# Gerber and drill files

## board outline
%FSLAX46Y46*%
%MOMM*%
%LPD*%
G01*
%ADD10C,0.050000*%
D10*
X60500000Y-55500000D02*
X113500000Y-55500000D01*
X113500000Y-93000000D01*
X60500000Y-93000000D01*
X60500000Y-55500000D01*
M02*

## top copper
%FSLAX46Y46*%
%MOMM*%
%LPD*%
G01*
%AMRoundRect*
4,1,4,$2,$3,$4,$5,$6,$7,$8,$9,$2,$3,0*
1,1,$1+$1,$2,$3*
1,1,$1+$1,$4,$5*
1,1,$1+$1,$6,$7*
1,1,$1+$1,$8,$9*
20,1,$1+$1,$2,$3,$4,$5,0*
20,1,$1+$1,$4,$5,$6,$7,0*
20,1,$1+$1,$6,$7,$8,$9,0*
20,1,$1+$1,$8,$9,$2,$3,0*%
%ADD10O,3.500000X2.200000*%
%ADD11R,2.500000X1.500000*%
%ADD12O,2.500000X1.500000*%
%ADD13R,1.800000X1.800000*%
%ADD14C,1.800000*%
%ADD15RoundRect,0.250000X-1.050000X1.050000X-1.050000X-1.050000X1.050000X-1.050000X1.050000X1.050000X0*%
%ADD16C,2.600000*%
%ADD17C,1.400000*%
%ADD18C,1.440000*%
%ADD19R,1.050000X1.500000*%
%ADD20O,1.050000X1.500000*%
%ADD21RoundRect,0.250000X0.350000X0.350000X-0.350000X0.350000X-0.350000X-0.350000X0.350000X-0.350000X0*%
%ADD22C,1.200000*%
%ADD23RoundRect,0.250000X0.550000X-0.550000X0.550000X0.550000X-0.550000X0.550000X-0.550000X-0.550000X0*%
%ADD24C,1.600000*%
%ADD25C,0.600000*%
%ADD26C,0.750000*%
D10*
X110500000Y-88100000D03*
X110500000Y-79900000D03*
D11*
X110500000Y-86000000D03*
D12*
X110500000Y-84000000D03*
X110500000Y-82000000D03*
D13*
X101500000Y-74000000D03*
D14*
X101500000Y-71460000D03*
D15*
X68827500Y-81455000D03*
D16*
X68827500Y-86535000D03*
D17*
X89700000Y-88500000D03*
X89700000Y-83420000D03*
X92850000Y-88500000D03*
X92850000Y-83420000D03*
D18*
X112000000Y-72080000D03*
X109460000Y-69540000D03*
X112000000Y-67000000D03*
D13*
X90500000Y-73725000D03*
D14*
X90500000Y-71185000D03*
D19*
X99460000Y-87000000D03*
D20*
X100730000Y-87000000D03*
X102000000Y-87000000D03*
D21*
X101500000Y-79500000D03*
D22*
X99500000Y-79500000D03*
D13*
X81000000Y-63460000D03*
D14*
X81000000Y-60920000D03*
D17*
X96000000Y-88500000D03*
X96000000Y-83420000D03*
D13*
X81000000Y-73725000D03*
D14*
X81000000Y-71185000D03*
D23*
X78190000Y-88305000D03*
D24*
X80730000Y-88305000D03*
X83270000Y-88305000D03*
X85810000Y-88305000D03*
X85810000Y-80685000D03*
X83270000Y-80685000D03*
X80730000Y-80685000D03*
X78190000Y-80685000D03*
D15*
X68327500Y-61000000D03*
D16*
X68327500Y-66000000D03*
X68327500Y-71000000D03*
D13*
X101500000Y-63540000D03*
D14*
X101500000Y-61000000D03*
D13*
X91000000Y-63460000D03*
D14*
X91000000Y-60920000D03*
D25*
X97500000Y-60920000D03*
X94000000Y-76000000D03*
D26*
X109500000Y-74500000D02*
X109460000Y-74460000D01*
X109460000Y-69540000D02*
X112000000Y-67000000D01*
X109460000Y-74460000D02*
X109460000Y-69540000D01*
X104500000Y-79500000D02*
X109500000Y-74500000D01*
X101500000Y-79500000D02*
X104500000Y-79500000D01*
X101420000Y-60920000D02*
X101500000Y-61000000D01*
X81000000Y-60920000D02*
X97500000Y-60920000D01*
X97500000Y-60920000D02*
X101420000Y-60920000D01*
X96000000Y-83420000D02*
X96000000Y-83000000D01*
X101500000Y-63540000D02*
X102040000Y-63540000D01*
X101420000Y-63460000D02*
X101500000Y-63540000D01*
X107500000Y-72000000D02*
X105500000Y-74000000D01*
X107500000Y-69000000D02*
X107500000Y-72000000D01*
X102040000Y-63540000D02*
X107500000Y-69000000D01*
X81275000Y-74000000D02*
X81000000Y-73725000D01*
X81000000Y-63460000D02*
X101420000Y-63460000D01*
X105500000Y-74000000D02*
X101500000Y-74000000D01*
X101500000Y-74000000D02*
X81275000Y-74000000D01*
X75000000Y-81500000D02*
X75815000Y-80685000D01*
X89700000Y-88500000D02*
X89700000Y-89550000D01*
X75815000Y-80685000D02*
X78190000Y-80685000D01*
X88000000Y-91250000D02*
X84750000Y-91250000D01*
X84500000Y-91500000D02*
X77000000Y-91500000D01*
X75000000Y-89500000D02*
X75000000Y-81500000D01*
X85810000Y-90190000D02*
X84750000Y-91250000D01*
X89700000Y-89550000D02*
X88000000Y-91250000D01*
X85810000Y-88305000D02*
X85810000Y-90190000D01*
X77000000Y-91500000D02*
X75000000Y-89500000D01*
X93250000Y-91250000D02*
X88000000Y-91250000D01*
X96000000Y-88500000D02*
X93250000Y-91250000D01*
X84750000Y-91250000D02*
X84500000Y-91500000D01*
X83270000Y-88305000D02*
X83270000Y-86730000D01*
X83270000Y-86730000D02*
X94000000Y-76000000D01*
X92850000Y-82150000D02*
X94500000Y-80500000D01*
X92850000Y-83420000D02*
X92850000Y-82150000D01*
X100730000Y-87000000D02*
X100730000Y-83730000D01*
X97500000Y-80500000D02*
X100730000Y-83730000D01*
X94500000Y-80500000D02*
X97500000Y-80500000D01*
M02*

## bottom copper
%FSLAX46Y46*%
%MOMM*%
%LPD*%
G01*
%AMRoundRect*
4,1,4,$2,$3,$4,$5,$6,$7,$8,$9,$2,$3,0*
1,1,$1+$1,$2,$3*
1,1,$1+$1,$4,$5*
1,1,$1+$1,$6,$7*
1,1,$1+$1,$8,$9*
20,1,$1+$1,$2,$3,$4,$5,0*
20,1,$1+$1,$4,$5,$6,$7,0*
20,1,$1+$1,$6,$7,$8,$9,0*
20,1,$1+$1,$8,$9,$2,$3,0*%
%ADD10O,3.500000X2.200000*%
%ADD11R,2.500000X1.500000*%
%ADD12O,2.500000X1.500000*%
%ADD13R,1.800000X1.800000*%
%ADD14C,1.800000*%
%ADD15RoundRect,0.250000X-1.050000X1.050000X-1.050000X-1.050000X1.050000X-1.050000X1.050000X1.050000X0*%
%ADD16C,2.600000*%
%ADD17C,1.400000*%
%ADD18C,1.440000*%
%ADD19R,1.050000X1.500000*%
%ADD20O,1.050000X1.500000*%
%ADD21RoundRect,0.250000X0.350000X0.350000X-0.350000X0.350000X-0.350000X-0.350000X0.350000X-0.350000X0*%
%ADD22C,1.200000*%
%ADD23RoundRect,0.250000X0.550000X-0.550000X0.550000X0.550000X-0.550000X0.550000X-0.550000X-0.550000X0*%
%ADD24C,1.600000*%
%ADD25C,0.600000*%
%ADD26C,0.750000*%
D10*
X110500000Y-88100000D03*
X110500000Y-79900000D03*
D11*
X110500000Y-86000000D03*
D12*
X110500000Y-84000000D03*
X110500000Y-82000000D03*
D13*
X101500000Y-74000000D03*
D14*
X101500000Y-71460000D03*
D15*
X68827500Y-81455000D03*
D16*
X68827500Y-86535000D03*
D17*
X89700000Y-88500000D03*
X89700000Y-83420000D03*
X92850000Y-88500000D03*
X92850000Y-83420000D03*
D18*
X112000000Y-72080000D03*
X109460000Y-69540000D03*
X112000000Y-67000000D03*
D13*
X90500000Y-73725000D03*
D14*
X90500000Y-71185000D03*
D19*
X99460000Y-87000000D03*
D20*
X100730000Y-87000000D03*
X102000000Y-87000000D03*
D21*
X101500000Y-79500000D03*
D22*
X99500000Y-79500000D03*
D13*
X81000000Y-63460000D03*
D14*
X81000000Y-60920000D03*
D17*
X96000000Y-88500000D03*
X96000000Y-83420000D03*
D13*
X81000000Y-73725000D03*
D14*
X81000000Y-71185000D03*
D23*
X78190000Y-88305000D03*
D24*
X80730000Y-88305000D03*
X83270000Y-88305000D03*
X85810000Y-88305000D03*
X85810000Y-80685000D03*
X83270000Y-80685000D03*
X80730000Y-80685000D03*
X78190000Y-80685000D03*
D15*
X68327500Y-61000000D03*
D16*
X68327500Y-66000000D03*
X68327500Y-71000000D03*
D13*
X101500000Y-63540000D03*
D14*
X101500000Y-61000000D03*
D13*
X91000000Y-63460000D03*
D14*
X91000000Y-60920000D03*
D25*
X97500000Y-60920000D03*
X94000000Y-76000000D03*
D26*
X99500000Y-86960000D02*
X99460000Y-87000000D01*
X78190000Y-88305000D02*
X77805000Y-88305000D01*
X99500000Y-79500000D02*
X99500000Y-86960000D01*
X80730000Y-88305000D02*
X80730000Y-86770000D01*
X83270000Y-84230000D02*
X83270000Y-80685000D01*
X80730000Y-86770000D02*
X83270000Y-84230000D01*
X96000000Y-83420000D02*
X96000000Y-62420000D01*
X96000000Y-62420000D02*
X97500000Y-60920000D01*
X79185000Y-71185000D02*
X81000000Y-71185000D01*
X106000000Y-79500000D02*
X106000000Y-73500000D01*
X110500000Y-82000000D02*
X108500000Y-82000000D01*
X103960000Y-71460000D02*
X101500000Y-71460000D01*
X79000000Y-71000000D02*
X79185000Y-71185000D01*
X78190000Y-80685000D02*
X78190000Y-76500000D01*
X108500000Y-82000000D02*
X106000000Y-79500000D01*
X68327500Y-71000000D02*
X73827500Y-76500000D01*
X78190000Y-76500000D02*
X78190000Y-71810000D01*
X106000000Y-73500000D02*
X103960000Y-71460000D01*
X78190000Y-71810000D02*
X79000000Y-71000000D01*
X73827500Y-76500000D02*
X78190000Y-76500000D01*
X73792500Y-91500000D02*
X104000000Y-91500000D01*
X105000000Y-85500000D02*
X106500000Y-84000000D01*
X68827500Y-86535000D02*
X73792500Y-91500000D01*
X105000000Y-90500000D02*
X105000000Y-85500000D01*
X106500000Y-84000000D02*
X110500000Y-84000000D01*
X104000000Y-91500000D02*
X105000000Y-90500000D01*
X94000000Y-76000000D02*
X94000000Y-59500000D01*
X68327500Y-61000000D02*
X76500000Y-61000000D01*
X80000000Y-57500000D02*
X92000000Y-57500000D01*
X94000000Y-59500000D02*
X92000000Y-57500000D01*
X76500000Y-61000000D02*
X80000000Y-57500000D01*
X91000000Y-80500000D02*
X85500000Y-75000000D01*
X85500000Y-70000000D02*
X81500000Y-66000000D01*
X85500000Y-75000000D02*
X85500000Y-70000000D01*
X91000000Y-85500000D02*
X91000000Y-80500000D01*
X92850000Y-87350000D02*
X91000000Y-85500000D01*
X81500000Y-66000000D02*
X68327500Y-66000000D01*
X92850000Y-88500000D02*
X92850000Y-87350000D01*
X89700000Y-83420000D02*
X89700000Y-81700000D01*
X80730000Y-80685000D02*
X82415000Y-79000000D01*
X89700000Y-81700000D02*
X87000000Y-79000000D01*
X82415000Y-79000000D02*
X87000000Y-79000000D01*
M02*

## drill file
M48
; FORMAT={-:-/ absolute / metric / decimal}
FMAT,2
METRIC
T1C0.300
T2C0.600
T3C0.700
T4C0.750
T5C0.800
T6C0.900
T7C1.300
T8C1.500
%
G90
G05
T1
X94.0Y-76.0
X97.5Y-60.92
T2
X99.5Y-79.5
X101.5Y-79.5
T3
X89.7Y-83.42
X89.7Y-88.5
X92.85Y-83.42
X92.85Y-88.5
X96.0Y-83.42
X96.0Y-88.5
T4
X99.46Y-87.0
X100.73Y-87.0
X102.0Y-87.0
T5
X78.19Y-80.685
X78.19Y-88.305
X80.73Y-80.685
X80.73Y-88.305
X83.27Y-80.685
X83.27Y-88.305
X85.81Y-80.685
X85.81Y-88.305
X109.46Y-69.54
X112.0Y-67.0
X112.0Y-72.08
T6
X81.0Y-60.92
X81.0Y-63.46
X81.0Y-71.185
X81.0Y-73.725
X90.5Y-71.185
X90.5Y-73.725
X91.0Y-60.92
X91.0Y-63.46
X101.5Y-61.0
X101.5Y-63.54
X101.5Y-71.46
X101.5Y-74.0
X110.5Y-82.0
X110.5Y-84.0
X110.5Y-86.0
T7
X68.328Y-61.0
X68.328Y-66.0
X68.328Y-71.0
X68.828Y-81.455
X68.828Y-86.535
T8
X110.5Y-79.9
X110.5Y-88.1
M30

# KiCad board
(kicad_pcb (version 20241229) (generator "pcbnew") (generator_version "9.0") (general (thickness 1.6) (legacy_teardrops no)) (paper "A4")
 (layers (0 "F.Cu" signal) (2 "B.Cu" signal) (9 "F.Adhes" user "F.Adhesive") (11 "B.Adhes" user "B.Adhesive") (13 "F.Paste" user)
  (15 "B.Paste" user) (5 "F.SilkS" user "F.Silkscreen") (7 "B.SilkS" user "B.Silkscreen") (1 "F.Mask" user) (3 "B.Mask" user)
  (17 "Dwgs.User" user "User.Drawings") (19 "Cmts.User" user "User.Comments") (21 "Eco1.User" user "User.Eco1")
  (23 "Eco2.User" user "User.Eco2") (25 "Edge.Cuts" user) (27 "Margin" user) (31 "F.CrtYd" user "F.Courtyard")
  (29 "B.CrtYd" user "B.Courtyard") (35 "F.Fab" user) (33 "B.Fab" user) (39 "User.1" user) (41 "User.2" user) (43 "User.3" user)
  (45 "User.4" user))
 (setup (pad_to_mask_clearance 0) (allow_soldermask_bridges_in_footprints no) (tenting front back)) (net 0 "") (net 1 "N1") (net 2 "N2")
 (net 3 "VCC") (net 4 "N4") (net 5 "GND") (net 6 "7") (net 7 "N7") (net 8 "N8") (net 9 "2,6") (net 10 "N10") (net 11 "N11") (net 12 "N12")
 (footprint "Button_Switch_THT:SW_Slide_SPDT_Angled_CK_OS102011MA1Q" (layer "F.Cu") (at 110.5 86 90)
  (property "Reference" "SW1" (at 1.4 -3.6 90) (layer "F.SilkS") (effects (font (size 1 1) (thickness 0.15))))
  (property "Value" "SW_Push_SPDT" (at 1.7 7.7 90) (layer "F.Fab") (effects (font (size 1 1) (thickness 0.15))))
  (pad "" thru_hole oval (at -2.1 0 90) (size 2.2 3.5) (drill 1.5) (layers "*.Cu" "*.Mask") (remove_unused_layers no))
  (pad "" thru_hole oval (at 6.1 0 90) (size 2.2 3.5) (drill 1.5) (layers "*.Cu" "*.Mask") (remove_unused_layers no))
  (pad "1" thru_hole rect (at 0 0 90) (size 1.5 2.5) (drill 0.9) (layers "*.Cu" "*.Mask") (remove_unused_layers no) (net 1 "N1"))
  (pad "2" thru_hole oval (at 2 0 90) (size 1.5 2.5) (drill 0.9) (layers "*.Cu" "*.Mask") (remove_unused_layers no) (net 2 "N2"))
  (pad "3" thru_hole oval (at 4 0 90) (size 1.5 2.5) (drill 0.9) (layers "*.Cu" "*.Mask") (remove_unused_layers no) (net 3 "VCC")))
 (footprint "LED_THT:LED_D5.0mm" (layer "F.Cu") (at 101.5 74 90)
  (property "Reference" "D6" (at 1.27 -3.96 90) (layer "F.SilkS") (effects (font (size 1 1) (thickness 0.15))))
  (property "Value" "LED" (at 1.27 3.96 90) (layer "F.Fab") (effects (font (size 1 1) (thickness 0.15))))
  (pad "1" thru_hole rect (at 0 0 90) (size 1.8 1.8) (drill 0.9) (layers "*.Cu" "*.Mask") (remove_unused_layers no) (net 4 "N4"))
  (pad "2" thru_hole circle (at 2.54 0 90) (size 1.8 1.8) (drill 0.9) (layers "*.Cu" "*.Mask") (remove_unused_layers no) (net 3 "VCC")))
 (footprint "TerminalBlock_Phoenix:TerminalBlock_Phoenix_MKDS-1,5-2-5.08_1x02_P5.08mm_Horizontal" (layer "F.Cu") (at 68.8275 81.455 -90)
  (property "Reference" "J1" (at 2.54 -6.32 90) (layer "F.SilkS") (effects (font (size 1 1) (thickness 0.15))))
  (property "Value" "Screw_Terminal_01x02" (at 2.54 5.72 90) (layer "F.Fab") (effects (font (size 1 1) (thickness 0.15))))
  (pad "1" thru_hole roundrect (at 0 0 270) (size 2.6 2.6) (drill 1.3) (layers "*.Cu" "*.Mask") (remove_unused_layers no)
   (roundrect_rratio 0.096154) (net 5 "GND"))
  (pad "2" thru_hole circle (at 5.08 0 270) (size 2.6 2.6) (drill 1.3) (layers "*.Cu" "*.Mask") (remove_unused_layers no) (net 2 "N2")))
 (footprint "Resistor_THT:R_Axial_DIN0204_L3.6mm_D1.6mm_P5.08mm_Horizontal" (layer "F.Cu") (at 89.7 88.5 90)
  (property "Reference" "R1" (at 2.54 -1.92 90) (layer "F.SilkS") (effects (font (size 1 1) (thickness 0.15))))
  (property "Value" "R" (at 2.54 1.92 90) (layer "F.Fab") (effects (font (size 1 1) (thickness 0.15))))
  (pad "1" thru_hole circle (at 0 0 90) (size 1.4 1.4) (drill 0.7) (layers "*.Cu" "*.Mask") (remove_unused_layers no) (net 3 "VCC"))
  (pad "2" thru_hole circle (at 5.08 0 90) (size 1.4 1.4) (drill 0.7) (layers "*.Cu" "*.Mask") (remove_unused_layers no) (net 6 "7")))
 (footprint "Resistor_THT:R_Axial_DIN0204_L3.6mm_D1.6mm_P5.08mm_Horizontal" (layer "F.Cu") (at 92.85 88.5 90)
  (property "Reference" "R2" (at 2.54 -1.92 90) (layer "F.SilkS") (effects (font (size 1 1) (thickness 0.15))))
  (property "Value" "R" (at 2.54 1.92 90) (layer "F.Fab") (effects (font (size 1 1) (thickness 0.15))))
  (pad "1" thru_hole circle (at 0 0 90) (size 1.4 1.4) (drill 0.7) (layers "*.Cu" "*.Mask") (remove_unused_layers no) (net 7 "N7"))
  (pad "2" thru_hole circle (at 5.08 0 90) (size 1.4 1.4) (drill 0.7) (layers "*.Cu" "*.Mask") (remove_unused_layers no) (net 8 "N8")))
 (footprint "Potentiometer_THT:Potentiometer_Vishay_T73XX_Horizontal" (layer "F.Cu") (at 112 72.08 180)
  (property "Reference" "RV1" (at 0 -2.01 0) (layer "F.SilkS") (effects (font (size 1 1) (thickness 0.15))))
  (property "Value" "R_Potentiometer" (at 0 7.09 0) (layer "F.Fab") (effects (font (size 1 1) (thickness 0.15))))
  (pad "1" thru_hole circle (at 0 0 180) (size 1.44 1.44) (drill 0.8) (layers "*.Cu" "*.Mask") (remove_unused_layers no) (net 6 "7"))
  (pad "2" thru_hole circle (at 2.54 2.54 180) (size 1.44 1.44) (drill 0.8) (layers "*.Cu" "*.Mask") (remove_unused_layers no) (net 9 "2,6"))
  (pad "3" thru_hole circle (at 0 5.08 180) (size 1.44 1.44) (drill 0.8) (layers "*.Cu" "*.Mask") (remove_unused_layers no) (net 9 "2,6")))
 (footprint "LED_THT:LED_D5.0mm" (layer "F.Cu") (at 90.5 73.725 90)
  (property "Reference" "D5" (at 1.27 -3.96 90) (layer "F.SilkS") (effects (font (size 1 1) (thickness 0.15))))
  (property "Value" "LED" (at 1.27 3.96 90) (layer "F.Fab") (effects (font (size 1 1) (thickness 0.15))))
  (pad "1" thru_hole rect (at 0 0 90) (size 1.8 1.8) (drill 0.9) (layers "*.Cu" "*.Mask") (remove_unused_layers no) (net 4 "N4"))
  (pad "2" thru_hole circle (at 2.54 0 90) (size 1.8 1.8) (drill 0.9) (layers "*.Cu" "*.Mask") (remove_unused_layers no) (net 3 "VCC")))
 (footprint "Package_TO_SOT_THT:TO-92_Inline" (layer "F.Cu") (at 99.46 87)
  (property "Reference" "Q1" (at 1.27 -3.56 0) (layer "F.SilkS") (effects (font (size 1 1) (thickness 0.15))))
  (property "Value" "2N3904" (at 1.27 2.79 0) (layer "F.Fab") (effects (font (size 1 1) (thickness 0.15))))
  (pad "1" thru_hole rect (at 0 0) (size 1.05 1.5) (drill 0.75) (layers "*.Cu" "*.Mask") (remove_unused_layers no) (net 5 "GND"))
  (pad "2" thru_hole oval (at 1.27 0) (size 1.05 1.5) (drill 0.75) (layers "*.Cu" "*.Mask") (remove_unused_layers no) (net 8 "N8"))
  (pad "3" thru_hole oval (at 2.54 0) (size 1.05 1.5) (drill 0.75) (layers "*.Cu" "*.Mask") (remove_unused_layers no) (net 4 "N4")))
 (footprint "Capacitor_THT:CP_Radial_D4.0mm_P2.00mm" (layer "F.Cu") (at 101.5 79.5 180)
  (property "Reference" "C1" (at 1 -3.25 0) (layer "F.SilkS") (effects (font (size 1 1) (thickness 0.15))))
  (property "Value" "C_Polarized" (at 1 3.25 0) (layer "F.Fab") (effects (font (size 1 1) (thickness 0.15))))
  (pad "1" thru_hole roundrect (at 0 0 180) (size 1.2 1.2) (drill 0.6) (layers "*.Cu" "*.Mask") (remove_unused_layers no)
   (roundrect_rratio 0.208333) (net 9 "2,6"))
  (pad "2" thru_hole circle (at 2 0 180) (size 1.2 1.2) (drill 0.6) (layers "*.Cu" "*.Mask") (remove_unused_layers no) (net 5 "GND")))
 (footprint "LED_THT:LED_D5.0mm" (layer "F.Cu") (at 81 63.46 90)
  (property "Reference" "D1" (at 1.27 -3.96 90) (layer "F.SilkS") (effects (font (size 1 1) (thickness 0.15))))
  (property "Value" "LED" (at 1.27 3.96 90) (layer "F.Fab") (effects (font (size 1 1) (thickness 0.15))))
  (pad "1" thru_hole rect (at 0 0 90) (size 1.8 1.8) (drill 0.9) (layers "*.Cu" "*.Mask") (remove_unused_layers no) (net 4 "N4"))
  (pad "2" thru_hole circle (at 2.54 0 90) (size 1.8 1.8) (drill 0.9) (layers "*.Cu" "*.Mask") (remove_unused_layers no) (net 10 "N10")))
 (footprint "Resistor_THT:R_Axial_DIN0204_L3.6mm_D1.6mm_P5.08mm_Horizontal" (layer "F.Cu") (at 96 88.5 90)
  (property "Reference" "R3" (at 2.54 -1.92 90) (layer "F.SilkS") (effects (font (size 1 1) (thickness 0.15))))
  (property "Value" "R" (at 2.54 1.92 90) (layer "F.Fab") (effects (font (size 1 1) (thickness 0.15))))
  (pad "1" thru_hole circle (at 0 0 90) (size 1.4 1.4) (drill 0.7) (layers "*.Cu" "*.Mask") (remove_unused_layers no) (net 3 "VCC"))
  (pad "2" thru_hole circle (at 5.08 0 90) (size 1.4 1.4) (drill 0.7) (layers "*.Cu" "*.Mask") (remove_unused_layers no) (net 10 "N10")))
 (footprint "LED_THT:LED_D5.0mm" (layer "F.Cu") (at 81 73.725 90)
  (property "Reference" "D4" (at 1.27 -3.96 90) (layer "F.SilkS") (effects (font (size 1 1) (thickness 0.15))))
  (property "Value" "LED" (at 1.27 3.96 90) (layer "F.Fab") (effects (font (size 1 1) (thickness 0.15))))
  (pad "1" thru_hole rect (at 0 0 90) (size 1.8 1.8) (drill 0.9) (layers "*.Cu" "*.Mask") (remove_unused_layers no) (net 4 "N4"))
  (pad "2" thru_hole circle (at 2.54 0 90) (size 1.8 1.8) (drill 0.9) (layers "*.Cu" "*.Mask") (remove_unused_layers no) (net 3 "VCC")))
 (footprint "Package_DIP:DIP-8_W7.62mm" (layer "F.Cu") (at 78.19 88.305 90)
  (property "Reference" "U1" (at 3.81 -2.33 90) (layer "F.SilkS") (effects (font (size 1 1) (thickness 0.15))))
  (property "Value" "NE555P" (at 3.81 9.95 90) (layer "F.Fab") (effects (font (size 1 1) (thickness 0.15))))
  (pad "1" thru_hole roundrect (at 0 0 90) (size 1.6 1.6) (drill 0.8) (layers "*.Cu" "*.Mask") (remove_unused_layers no)
   (roundrect_rratio 0.15625) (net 5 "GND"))
  (pad "2" thru_hole circle (at 0 2.54 90) (size 1.6 1.6) (drill 0.8) (layers "*.Cu" "*.Mask") (remove_unused_layers no) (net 9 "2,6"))
  (pad "3" thru_hole circle (at 0 5.08 90) (size 1.6 1.6) (drill 0.8) (layers "*.Cu" "*.Mask") (remove_unused_layers no) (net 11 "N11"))
  (pad "4" thru_hole circle (at 0 7.62 90) (size 1.6 1.6) (drill 0.8) (layers "*.Cu" "*.Mask") (remove_unused_layers no) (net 3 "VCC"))
  (pad "5" thru_hole circle (at 7.62 7.62 90) (size 1.6 1.6) (drill 0.8) (layers "*.Cu" "*.Mask") (remove_unused_layers no) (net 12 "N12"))
  (pad "6" thru_hole circle (at 7.62 5.08 90) (size 1.6 1.6) (drill 0.8) (layers "*.Cu" "*.Mask") (remove_unused_layers no) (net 9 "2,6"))
  (pad "7" thru_hole circle (at 7.62 2.54 90) (size 1.6 1.6) (drill 0.8) (layers "*.Cu" "*.Mask") (remove_unused_layers no) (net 6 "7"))
  (pad "8" thru_hole circle (at 7.62 0 90) (size 1.6 1.6) (drill 0.8) (layers "*.Cu" "*.Mask") (remove_unused_layers no) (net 3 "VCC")))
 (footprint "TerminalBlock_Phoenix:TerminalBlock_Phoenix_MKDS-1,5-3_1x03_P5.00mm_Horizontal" (layer "F.Cu") (at 68.3275 61 -90)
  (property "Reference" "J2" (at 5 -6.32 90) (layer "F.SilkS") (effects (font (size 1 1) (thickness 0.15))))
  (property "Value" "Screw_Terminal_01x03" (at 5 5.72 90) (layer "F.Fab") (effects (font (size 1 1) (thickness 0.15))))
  (pad "1" thru_hole roundrect (at 0 0 270) (size 2.6 2.6) (drill 1.3) (layers "*.Cu" "*.Mask") (remove_unused_layers no)
   (roundrect_rratio 0.096154) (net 11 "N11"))
  (pad "2" thru_hole circle (at 5 0 270) (size 2.6 2.6) (drill 1.3) (layers "*.Cu" "*.Mask") (remove_unused_layers no) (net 7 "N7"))
  (pad "3" thru_hole circle (at 10 0 270) (size 2.6 2.6) (drill 1.3) (layers "*.Cu" "*.Mask") (remove_unused_layers no) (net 3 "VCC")))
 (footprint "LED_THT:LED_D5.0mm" (layer "F.Cu") (at 101.5 63.54 90)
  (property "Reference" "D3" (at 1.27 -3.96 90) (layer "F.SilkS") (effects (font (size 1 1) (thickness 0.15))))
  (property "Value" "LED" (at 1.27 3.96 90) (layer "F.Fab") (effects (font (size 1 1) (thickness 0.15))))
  (pad "1" thru_hole rect (at 0 0 90) (size 1.8 1.8) (drill 0.9) (layers "*.Cu" "*.Mask") (remove_unused_layers no) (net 4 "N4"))
  (pad "2" thru_hole circle (at 2.54 0 90) (size 1.8 1.8) (drill 0.9) (layers "*.Cu" "*.Mask") (remove_unused_layers no) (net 10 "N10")))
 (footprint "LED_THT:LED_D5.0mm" (layer "F.Cu") (at 91 63.46 90)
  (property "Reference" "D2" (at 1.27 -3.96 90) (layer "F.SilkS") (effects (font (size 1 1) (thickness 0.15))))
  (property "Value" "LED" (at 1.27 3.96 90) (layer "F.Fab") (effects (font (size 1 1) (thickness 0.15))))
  (pad "1" thru_hole rect (at 0 0 90) (size 1.8 1.8) (drill 0.9) (layers "*.Cu" "*.Mask") (remove_unused_layers no) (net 4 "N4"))
  (pad "2" thru_hole circle (at 2.54 0 90) (size 1.8 1.8) (drill 0.9) (layers "*.Cu" "*.Mask") (remove_unused_layers no) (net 10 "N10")))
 (gr_rect (start 60.5 55.5) (end 113.5 93) (stroke (width 0.05) (type default)) (fill no) (layer "Edge.Cuts"))
 (segment (start 99.5 86.96) (end 99.46 87) (width 0.75) (layer "B.Cu") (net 5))
 (segment (start 78.19 88.305) (end 77.805 88.305) (width 0.75) (layer "B.Cu") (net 5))
 (segment (start 99.5 79.5) (end 99.5 86.96) (width 0.75) (layer "B.Cu") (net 5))
 (segment (start 109.5 74.5) (end 109.46 74.46) (width 0.75) (layer "F.Cu") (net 9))
 (segment (start 109.46 69.54) (end 112 67) (width 0.75) (layer "F.Cu") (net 9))
 (segment (start 109.46 74.46) (end 109.46 69.54) (width 0.75) (layer "F.Cu") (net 9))
 (segment (start 104.5 79.5) (end 109.5 74.5) (width 0.75) (layer "F.Cu") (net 9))
 (segment (start 101.5 79.5) (end 104.5 79.5) (width 0.75) (layer "F.Cu") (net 9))
 (segment (start 80.73 88.305) (end 80.73 86.77) (width 0.75) (layer "B.Cu") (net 9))
 (segment (start 83.27 84.23) (end 83.27 80.685) (width 0.75) (layer "B.Cu") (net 9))
 (segment (start 80.73 86.77) (end 83.27 84.23) (width 0.75) (layer "B.Cu") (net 9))
 (segment (start 101.42 60.92) (end 101.5 61) (width 0.75) (layer "F.Cu") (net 10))
 (segment (start 81 60.92) (end 97.5 60.92) (width 0.75) (layer "F.Cu") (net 10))
 (segment (start 97.5 60.92) (end 101.42 60.92) (width 0.75) (layer "F.Cu") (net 10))
 (segment (start 96 83.42) (end 96 83) (width 0.75) (layer "F.Cu") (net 10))
 (via (at 97.5 60.92) (size 0.6) (drill 0.3) (layers "F.Cu" "B.Cu") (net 10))
 (segment (start 96 83.42) (end 96 62.42) (width 0.75) (layer "B.Cu") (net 10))
 (segment (start 96 62.42) (end 97.5 60.92) (width 0.75) (layer "B.Cu") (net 10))
 (segment (start 101.5 63.54) (end 102.04 63.54) (width 0.75) (layer "F.Cu") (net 4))
 (segment (start 101.42 63.46) (end 101.5 63.54) (width 0.75) (layer "F.Cu") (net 4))
 (segment (start 107.5 72) (end 105.5 74) (width 0.75) (layer "F.Cu") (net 4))
 (segment (start 107.5 69) (end 107.5 72) (width 0.75) (layer "F.Cu") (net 4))
 (segment (start 102.04 63.54) (end 107.5 69) (width 0.75) (layer "F.Cu") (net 4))
 (segment (start 81.275 74) (end 81 73.725) (width 0.75) (layer "F.Cu") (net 4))
 (segment (start 81 63.46) (end 101.42 63.46) (width 0.75) (layer "F.Cu") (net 4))
 (segment (start 105.5 74) (end 101.5 74) (width 0.75) (layer "F.Cu") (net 4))
 (segment (start 101.5 74) (end 81.275 74) (width 0.75) (layer "F.Cu") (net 4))
 (segment (start 75 81.5) (end 75.815 80.685) (width 0.75) (layer "F.Cu") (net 3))
 (segment (start 89.7 88.5) (end 89.7 89.55) (width 0.75) (layer "F.Cu") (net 3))
 (segment (start 75.815 80.685) (end 78.19 80.685) (width 0.75) (layer "F.Cu") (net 3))
 (segment (start 88 91.25) (end 84.75 91.25) (width 0.75) (layer "F.Cu") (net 3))
 (segment (start 84.5 91.5) (end 77 91.5) (width 0.75) (layer "F.Cu") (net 3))
 (segment (start 75 89.5) (end 75 81.5) (width 0.75) (layer "F.Cu") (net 3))
 (segment (start 85.81 90.19) (end 84.75 91.25) (width 0.75) (layer "F.Cu") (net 3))
 (segment (start 89.7 89.55) (end 88 91.25) (width 0.75) (layer "F.Cu") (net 3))
 (segment (start 85.81 88.305) (end 85.81 90.19) (width 0.75) (layer "F.Cu") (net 3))
 (segment (start 77 91.5) (end 75 89.5) (width 0.75) (layer "F.Cu") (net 3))
 (segment (start 93.25 91.25) (end 88 91.25) (width 0.75) (layer "F.Cu") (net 3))
 (segment (start 96 88.5) (end 93.25 91.25) (width 0.75) (layer "F.Cu") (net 3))
 (segment (start 84.75 91.25) (end 84.5 91.5) (width 0.75) (layer "F.Cu") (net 3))
 (segment (start 79.185 71.185) (end 81 71.185) (width 0.75) (layer "B.Cu") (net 3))
 (segment (start 106 79.5) (end 106 73.5) (width 0.75) (layer "B.Cu") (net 3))
 (segment (start 110.5 82) (end 108.5 82) (width 0.75) (layer "B.Cu") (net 3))
 (segment (start 103.96 71.46) (end 101.5 71.46) (width 0.75) (layer "B.Cu") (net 3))
 (segment (start 79 71) (end 79.185 71.185) (width 0.75) (layer "B.Cu") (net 3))
 (segment (start 78.19 80.685) (end 78.19 76.5) (width 0.75) (layer "B.Cu") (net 3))
 (segment (start 108.5 82) (end 106 79.5) (width 0.75) (layer "B.Cu") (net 3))
 (segment (start 68.3275 71) (end 73.8275 76.5) (width 0.75) (layer "B.Cu") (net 3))
 (segment (start 78.19 76.5) (end 78.19 71.81) (width 0.75) (layer "B.Cu") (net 3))
 (segment (start 106 73.5) (end 103.96 71.46) (width 0.75) (layer "B.Cu") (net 3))
 (segment (start 78.19 71.81) (end 79 71) (width 0.75) (layer "B.Cu") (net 3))
 (segment (start 73.8275 76.5) (end 78.19 76.5) (width 0.75) (layer "B.Cu") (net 3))
 (segment (start 73.7925 91.5) (end 104 91.5) (width 0.75) (layer "B.Cu") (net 2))
 (segment (start 105 85.5) (end 106.5 84) (width 0.75) (layer "B.Cu") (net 2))
 (segment (start 68.8275 86.535) (end 73.7925 91.5) (width 0.75) (layer "B.Cu") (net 2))
 (segment (start 105 90.5) (end 105 85.5) (width 0.75) (layer "B.Cu") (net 2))
 (segment (start 106.5 84) (end 110.5 84) (width 0.75) (layer "B.Cu") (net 2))
 (segment (start 104 91.5) (end 105 90.5) (width 0.75) (layer "B.Cu") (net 2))
 (segment (start 83.27 88.305) (end 83.27 86.73) (width 0.75) (layer "F.Cu") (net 11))
 (segment (start 83.27 86.73) (end 94 76) (width 0.75) (layer "F.Cu") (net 11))
 (via (at 94 76) (size 0.6) (drill 0.3) (layers "F.Cu" "B.Cu") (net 11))
 (segment (start 94 76) (end 94 59.5) (width 0.75) (layer "B.Cu") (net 11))
 (segment (start 68.3275 61) (end 76.5 61) (width 0.75) (layer "B.Cu") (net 11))
 (segment (start 80 57.5) (end 92 57.5) (width 0.75) (layer "B.Cu") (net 11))
 (segment (start 94 59.5) (end 92 57.5) (width 0.75) (layer "B.Cu") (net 11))
 (segment (start 76.5 61) (end 80 57.5) (width 0.75) (layer "B.Cu") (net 11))
 (segment (start 91 80.5) (end 85.5 75) (width 0.75) (layer "B.Cu") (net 7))
 (segment (start 85.5 70) (end 81.5 66) (width 0.75) (layer "B.Cu") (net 7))
 (segment (start 85.5 75) (end 85.5 70) (width 0.75) (layer "B.Cu") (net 7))
 (segment (start 91 85.5) (end 91 80.5) (width 0.75) (layer "B.Cu") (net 7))
 (segment (start 92.85 87.35) (end 91 85.5) (width 0.75) (layer "B.Cu") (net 7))
 (segment (start 81.5 66) (end 68.3275 66) (width 0.75) (layer "B.Cu") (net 7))
 (segment (start 92.85 88.5) (end 92.85 87.35) (width 0.75) (layer "B.Cu") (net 7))
 (segment (start 92.85 82.15) (end 94.5 80.5) (width 0.75) (layer "F.Cu") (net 8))
 (segment (start 92.85 83.42) (end 92.85 82.15) (width 0.75) (layer "F.Cu") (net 8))
 (segment (start 100.73 87) (end 100.73 83.73) (width 0.75) (layer "F.Cu") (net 8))
 (segment (start 97.5 80.5) (end 100.73 83.73) (width 0.75) (layer "F.Cu") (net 8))
 (segment (start 94.5 80.5) (end 97.5 80.5) (width 0.75) (layer "F.Cu") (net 8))
 (segment (start 89.7 83.42) (end 89.7 81.7) (width 0.75) (layer "B.Cu") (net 6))
 (segment (start 80.73 80.685) (end 82.415 79) (width 0.75) (layer "B.Cu") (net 6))
 (segment (start 89.7 81.7) (end 87 79) (width 0.75) (layer "B.Cu") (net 6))
 (segment (start 82.415 79) (end 87 79) (width 0.75) (layer "B.Cu") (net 6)))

